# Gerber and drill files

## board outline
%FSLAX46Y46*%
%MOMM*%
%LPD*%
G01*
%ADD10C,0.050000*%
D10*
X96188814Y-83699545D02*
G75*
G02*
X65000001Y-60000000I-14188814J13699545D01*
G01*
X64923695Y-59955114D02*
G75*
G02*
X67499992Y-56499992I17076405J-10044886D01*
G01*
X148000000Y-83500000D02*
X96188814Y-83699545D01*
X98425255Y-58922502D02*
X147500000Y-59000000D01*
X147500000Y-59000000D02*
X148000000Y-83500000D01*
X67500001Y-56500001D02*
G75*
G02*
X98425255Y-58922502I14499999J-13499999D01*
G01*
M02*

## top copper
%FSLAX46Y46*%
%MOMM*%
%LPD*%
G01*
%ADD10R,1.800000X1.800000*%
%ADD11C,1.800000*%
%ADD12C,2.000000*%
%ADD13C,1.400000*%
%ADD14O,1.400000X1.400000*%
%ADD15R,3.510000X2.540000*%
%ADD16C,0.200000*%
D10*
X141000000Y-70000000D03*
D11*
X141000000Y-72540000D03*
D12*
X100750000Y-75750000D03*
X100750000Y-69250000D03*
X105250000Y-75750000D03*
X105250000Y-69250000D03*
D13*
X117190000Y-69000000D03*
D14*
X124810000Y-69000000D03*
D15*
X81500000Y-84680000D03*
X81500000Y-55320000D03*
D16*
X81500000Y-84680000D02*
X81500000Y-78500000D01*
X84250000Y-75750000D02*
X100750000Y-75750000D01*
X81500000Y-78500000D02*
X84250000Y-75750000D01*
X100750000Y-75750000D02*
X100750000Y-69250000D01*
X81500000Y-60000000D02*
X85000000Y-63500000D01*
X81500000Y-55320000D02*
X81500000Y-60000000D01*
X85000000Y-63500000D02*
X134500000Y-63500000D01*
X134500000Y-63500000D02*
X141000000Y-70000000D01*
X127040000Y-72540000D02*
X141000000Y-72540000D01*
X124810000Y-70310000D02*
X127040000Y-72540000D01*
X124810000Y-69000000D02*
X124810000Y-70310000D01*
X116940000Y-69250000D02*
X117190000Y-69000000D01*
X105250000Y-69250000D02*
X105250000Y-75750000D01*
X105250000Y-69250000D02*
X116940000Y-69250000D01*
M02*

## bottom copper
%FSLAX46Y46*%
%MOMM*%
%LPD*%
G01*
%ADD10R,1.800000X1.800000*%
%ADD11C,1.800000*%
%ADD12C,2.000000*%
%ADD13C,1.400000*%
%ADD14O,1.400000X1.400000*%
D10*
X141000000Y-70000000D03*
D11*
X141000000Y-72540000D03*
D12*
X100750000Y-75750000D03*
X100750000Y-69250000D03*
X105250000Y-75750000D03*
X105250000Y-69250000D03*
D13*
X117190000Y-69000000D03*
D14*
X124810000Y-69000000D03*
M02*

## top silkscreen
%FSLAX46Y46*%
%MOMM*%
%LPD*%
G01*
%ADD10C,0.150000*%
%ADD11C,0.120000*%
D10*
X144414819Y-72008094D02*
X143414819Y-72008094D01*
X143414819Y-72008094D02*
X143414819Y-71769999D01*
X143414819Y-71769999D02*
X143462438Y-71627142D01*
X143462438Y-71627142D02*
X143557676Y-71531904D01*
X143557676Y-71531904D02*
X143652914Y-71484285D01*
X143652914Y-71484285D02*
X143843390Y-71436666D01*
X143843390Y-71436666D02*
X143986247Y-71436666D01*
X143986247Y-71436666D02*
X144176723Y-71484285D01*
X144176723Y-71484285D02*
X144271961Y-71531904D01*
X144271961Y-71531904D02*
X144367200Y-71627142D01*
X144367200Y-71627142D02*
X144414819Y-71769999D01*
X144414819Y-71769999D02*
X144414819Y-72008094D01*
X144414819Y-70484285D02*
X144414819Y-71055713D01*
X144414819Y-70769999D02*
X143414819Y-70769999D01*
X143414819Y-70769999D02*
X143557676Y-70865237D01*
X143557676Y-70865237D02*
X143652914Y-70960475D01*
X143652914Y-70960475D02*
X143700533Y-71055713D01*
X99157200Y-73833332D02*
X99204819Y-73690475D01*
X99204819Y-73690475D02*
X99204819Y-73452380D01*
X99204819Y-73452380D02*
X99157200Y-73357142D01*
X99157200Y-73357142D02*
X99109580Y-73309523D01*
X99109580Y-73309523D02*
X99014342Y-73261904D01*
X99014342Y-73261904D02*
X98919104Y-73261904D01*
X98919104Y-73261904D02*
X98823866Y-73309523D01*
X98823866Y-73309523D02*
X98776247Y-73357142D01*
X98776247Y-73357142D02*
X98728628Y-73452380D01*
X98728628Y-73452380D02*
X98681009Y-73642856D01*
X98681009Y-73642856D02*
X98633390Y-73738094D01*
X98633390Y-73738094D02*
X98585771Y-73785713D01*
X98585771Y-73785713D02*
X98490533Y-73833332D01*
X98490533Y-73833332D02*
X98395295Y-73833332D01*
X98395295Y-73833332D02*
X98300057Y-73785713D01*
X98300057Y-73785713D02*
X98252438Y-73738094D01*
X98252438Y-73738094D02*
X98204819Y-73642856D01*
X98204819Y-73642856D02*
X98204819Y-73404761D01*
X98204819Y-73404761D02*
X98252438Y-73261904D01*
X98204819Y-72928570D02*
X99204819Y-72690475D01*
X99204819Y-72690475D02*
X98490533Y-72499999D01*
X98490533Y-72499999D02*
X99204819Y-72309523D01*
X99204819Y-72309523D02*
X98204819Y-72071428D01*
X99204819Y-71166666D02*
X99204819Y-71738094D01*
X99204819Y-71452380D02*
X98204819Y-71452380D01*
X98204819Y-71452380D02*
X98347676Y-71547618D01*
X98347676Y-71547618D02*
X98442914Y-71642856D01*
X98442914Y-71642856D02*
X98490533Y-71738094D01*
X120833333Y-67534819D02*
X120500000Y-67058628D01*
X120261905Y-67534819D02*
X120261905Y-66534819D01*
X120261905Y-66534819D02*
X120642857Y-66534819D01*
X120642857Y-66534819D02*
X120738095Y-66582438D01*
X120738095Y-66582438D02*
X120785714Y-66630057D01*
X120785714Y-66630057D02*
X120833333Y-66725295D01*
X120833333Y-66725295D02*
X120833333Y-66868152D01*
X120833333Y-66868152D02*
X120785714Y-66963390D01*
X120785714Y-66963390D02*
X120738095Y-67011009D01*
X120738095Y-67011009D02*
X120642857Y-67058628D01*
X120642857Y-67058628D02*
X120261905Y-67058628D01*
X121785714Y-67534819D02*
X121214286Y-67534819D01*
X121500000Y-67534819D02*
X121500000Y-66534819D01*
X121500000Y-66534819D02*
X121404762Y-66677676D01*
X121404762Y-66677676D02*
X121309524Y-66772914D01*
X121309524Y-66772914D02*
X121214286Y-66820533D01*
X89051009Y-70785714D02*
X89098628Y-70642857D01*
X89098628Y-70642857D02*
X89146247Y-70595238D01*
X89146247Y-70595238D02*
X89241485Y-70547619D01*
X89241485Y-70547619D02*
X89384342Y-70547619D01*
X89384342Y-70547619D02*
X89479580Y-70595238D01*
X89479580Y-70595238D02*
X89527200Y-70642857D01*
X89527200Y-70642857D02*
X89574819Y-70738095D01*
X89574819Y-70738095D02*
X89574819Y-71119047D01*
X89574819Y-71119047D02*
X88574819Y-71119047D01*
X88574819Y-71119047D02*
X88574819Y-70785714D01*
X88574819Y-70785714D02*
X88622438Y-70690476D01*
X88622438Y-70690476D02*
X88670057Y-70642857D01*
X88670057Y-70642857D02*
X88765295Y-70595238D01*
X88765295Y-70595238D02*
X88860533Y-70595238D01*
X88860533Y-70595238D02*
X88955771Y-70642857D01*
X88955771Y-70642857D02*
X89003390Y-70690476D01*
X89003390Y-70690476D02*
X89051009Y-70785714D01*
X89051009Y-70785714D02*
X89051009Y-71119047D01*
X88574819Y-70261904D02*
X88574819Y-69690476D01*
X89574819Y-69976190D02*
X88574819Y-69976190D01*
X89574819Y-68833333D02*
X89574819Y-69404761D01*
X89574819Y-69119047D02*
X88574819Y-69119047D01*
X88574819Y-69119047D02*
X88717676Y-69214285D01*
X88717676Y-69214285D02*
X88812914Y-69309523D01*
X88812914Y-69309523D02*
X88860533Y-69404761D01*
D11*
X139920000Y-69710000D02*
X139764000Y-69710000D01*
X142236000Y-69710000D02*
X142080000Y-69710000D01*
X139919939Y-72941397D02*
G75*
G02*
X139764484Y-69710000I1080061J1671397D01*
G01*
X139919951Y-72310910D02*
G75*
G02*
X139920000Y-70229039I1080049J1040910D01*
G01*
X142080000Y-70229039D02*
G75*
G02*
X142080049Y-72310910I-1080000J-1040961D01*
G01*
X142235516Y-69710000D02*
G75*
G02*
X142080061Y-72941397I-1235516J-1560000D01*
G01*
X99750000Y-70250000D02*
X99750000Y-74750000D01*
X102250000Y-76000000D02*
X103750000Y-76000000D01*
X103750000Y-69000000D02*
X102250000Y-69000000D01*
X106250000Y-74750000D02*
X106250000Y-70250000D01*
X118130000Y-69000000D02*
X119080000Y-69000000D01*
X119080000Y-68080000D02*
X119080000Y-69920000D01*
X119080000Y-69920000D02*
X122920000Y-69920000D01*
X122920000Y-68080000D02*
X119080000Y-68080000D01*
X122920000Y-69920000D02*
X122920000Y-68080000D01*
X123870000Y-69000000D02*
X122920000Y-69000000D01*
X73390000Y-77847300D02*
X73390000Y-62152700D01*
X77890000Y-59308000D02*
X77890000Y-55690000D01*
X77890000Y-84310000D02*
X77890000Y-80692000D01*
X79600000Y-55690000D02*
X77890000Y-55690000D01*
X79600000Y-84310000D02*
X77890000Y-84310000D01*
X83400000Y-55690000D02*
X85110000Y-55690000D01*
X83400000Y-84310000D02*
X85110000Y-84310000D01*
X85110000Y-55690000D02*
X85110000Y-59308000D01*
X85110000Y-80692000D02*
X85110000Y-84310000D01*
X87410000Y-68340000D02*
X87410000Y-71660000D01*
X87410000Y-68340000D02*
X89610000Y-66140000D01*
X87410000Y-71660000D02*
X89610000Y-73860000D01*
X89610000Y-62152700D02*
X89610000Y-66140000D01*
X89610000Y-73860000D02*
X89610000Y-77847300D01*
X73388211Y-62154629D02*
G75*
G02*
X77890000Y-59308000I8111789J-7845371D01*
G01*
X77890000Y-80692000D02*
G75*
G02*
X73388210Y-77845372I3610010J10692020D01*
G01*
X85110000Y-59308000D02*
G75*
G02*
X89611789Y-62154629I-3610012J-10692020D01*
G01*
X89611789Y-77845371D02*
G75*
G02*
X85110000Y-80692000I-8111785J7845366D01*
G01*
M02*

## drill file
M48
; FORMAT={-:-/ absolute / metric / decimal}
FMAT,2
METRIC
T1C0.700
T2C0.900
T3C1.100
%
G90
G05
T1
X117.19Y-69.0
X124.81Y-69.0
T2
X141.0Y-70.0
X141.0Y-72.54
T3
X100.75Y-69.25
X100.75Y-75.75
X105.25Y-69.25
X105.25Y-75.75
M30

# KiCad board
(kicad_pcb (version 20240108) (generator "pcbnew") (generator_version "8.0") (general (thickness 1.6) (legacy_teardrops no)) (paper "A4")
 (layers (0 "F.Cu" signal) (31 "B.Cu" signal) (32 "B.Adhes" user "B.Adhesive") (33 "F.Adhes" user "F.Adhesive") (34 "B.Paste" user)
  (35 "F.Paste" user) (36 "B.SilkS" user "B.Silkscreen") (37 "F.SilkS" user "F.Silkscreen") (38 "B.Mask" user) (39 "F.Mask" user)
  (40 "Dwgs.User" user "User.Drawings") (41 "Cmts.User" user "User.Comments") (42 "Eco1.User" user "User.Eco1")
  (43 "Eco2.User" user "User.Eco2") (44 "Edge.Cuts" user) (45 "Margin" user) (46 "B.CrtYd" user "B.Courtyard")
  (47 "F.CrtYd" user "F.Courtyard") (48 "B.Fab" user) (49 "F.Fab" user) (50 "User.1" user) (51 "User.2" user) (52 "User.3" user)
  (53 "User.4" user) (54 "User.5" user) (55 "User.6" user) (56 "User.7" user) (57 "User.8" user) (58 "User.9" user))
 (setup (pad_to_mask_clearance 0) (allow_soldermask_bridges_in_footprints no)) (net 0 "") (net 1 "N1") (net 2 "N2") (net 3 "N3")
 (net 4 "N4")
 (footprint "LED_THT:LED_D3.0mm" (layer "F.Cu") (at 141 70 -90)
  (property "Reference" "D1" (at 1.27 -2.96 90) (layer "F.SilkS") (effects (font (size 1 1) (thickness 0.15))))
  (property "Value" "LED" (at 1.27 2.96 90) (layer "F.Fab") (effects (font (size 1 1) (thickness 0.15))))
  (fp_line (start -0.29 1.08) (end -0.29 1.236) (stroke (width 0.12) (type solid)) (layer "F.SilkS"))
  (fp_line (start -0.29 -1.236) (end -0.29 -1.08) (stroke (width 0.12) (type solid)) (layer "F.SilkS"))
  (fp_arc (start 2.941397 1.080061) (mid 1.365624 1.987701) (end -0.29 1.235516) (stroke (width 0.12) (type solid)) (layer "F.SilkS"))
  (fp_arc (start 2.31091 1.080049) (mid 1.269965 1.5) (end 0.229039 1.08) (stroke (width 0.12) (type solid)) (layer "F.SilkS"))
  (fp_arc (start 0.229039 -1.08) (mid 1.269965 -1.5) (end 2.31091 -1.080049) (stroke (width 0.12) (type solid)) (layer "F.SilkS"))
  (fp_arc (start -0.29 -1.235516) (mid 1.365624 -1.987701) (end 2.941397 -1.080061) (stroke (width 0.12) (type solid)) (layer "F.SilkS"))
  (pad "1" thru_hole rect (at 0 0 270) (size 1.8 1.8) (drill 0.9) (layers "*.Cu" "*.Mask") (remove_unused_layers no) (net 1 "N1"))
  (pad "2" thru_hole circle (at 2.54 0 270) (size 1.8 1.8) (drill 0.9) (layers "*.Cu" "*.Mask") (remove_unused_layers no) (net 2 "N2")))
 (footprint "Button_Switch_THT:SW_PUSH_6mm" (layer "F.Cu") (at 100.75 75.75 90)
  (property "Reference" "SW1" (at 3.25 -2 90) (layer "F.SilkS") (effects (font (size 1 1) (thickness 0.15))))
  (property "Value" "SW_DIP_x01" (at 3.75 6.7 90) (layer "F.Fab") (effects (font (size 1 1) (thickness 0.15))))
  (fp_line (start 5.5 -1) (end 1 -1) (stroke (width 0.12) (type solid)) (layer "F.SilkS"))
  (fp_line (start -0.25 1.5) (end -0.25 3) (stroke (width 0.12) (type solid)) (layer "F.SilkS"))
  (fp_line (start 6.75 3) (end 6.75 1.5) (stroke (width 0.12) (type solid)) (layer "F.SilkS"))
  (fp_line (start 1 5.5) (end 5.5 5.5) (stroke (width 0.12) (type solid)) (layer "F.SilkS"))
  (pad "1" thru_hole circle (at 0 0 180) (size 2 2) (drill 1.1) (layers "*.Cu" "*.Mask") (remove_unused_layers no) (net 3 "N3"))
  (pad "1" thru_hole circle (at 6.5 0 180) (size 2 2) (drill 1.1) (layers "*.Cu" "*.Mask") (remove_unused_layers no) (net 3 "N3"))
  (pad "2" thru_hole circle (at 0 4.5 180) (size 2 2) (drill 1.1) (layers "*.Cu" "*.Mask") (remove_unused_layers no) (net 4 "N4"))
  (pad "2" thru_hole circle (at 6.5 4.5 180) (size 2 2) (drill 1.1) (layers "*.Cu" "*.Mask") (remove_unused_layers no) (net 4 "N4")))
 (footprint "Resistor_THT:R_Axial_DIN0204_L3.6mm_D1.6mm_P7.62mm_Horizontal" (layer "F.Cu") (at 117.19 69)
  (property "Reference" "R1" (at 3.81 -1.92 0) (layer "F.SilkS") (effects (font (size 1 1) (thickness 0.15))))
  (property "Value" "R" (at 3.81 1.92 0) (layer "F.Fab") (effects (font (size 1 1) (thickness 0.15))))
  (fp_line (start 0.94 0) (end 1.89 0) (stroke (width 0.12) (type solid)) (layer "F.SilkS"))
  (fp_line (start 1.89 -0.92) (end 1.89 0.92) (stroke (width 0.12) (type solid)) (layer "F.SilkS"))
  (fp_line (start 1.89 0.92) (end 5.73 0.92) (stroke (width 0.12) (type solid)) (layer "F.SilkS"))
  (fp_line (start 5.73 -0.92) (end 1.89 -0.92) (stroke (width 0.12) (type solid)) (layer "F.SilkS"))
  (fp_line (start 5.73 0.92) (end 5.73 -0.92) (stroke (width 0.12) (type solid)) (layer "F.SilkS"))
  (fp_line (start 6.68 0) (end 5.73 0) (stroke (width 0.12) (type solid)) (layer "F.SilkS"))
  (pad "1" thru_hole circle (at 0 0) (size 1.4 1.4) (drill 0.7) (layers "*.Cu" "*.Mask") (remove_unused_layers no) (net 4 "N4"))
  (pad "2" thru_hole oval (at 7.62 0) (size 1.4 1.4) (drill 0.7) (layers "*.Cu" "*.Mask") (remove_unused_layers no) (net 2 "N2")))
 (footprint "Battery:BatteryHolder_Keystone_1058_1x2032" (layer "F.Cu") (at 81.5 70 90)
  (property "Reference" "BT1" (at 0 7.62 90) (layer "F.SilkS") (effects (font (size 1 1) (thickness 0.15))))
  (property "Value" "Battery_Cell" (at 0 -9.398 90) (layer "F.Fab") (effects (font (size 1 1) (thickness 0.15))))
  (fp_line (start -7.8473 -8.11) (end 7.8473 -8.11) (stroke (width 0.12) (type solid)) (layer "F.SilkS"))
  (fp_line (start 10.692 -3.61) (end 14.31 -3.61) (stroke (width 0.12) (type solid)) (layer "F.SilkS"))
  (fp_line (start -14.31 -3.61) (end -10.692 -3.61) (stroke (width 0.12) (type solid)) (layer "F.SilkS"))
  (fp_line (start 14.31 -1.9) (end 14.31 -3.61) (stroke (width 0.12) (type solid)) (layer "F.SilkS"))
  (fp_line (start -14.31 -1.9) (end -14.31 -3.61) (stroke (width 0.12) (type solid)) (layer "F.SilkS"))
  (fp_line (start 14.31 1.9) (end 14.31 3.61) (stroke (width 0.12) (type solid)) (layer "F.SilkS"))
  (fp_line (start -14.31 1.9) (end -14.31 3.61) (stroke (width 0.12) (type solid)) (layer "F.SilkS"))
  (fp_line (start 14.31 3.61) (end 10.692 3.61) (stroke (width 0.12) (type solid)) (layer "F.SilkS"))
  (fp_line (start -10.692 3.61) (end -14.31 3.61) (stroke (width 0.12) (type solid)) (layer "F.SilkS"))
  (fp_line (start 1.66 5.91) (end -1.66 5.91) (stroke (width 0.12) (type solid)) (layer "F.SilkS"))
  (fp_line (start 1.66 5.91) (end 3.86 8.11) (stroke (width 0.12) (type solid)) (layer "F.SilkS"))
  (fp_line (start -1.66 5.91) (end -3.86 8.11) (stroke (width 0.12) (type solid)) (layer "F.SilkS"))
  (fp_line (start 7.8473 8.11) (end 3.86 8.11) (stroke (width 0.12) (type solid)) (layer "F.SilkS"))
  (fp_line (start -3.86 8.11) (end -7.8473 8.11) (stroke (width 0.12) (type solid)) (layer "F.SilkS"))
  (fp_arc (start 7.845371 -8.111789) (mid 9.538085 -6.031244) (end 10.692 -3.61) (stroke (width 0.12) (type solid)) (layer "F.SilkS"))
  (fp_arc (start -10.692 -3.61) (mid -9.538084 -6.031244) (end -7.845371 -8.111789) (stroke (width 0.12) (type solid)) (layer "F.SilkS"))
  (fp_arc (start 10.692 3.61) (mid 9.538084 6.031244) (end 7.845371 8.111789) (stroke (width 0.12) (type solid)) (layer "F.SilkS"))
  (fp_arc (start -7.845371 8.111789) (mid -9.538085 6.031244) (end -10.692 3.61) (stroke (width 0.12) (type solid)) (layer "F.SilkS"))
  (pad "1" smd rect (at -14.68 0 90) (size 2.54 3.51) (layers "F.Cu" "F.Paste" "F.Mask") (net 3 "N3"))
  (pad "2" smd rect (at 14.68 0 90) (size 2.54 3.51) (layers "F.Cu" "F.Paste" "F.Mask") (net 1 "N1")))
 (gr_arc (start 96.188814 83.699545) (mid 70.067155 85.703731) (end 65.000001 60) (stroke (width 0.05) (type default)) (layer "Edge.Cuts"))
 (gr_arc (start 64.923695 59.955114) (mid 66.117614 58.157292) (end 67.500001 56.500001) (stroke (width 0.05) (type default))
  (layer "Edge.Cuts"))
 (gr_line (start 148 83.5) (end 96.188814 83.699545) (stroke (width 0.05) (type default)) (layer "Edge.Cuts"))
 (gr_line (start 98.425255 58.922502) (end 147.5 59) (stroke (width 0.05) (type default)) (layer "Edge.Cuts"))
 (gr_line (start 147.5 59) (end 148 83.5) (stroke (width 0.05) (type default)) (layer "Edge.Cuts"))
 (gr_arc (start 67.500001 56.500001) (mid 83.547185 50.248895) (end 98.425255 58.922502) (stroke (width 0.05) (type default))
  (layer "Edge.Cuts"))
 (segment (start 81.5 84.68) (end 81.5 78.5) (width 0.2) (layer "F.Cu") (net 3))
 (segment (start 84.25 75.75) (end 100.75 75.75) (width 0.2) (layer "F.Cu") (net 3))
 (segment (start 81.5 78.5) (end 84.25 75.75) (width 0.2) (layer "F.Cu") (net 3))
 (segment (start 100.75 75.75) (end 100.75 69.25) (width 0.2) (layer "F.Cu") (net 3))
 (segment (start 81.5 60) (end 85 63.5) (width 0.2) (layer "F.Cu") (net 1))
 (segment (start 81.5 55.32) (end 81.5 60) (width 0.2) (layer "F.Cu") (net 1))
 (segment (start 85 63.5) (end 134.5 63.5) (width 0.2) (layer "F.Cu") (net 1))
 (segment (start 134.5 63.5) (end 141 70) (width 0.2) (layer "F.Cu") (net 1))
 (segment (start 127.04 72.54) (end 141 72.54) (width 0.2) (layer "F.Cu") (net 2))
 (segment (start 124.81 70.31) (end 127.04 72.54) (width 0.2) (layer "F.Cu") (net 2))
 (segment (start 124.81 69) (end 124.81 70.31) (width 0.2) (layer "F.Cu") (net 2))
 (segment (start 116.94 69.25) (end 117.19 69) (width 0.2) (layer "F.Cu") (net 4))
 (segment (start 105.25 69.25) (end 105.25 75.75) (width 0.2) (layer "F.Cu") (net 4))
 (segment (start 105.25 69.25) (end 116.94 69.25) (width 0.2) (layer "F.Cu") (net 4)))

